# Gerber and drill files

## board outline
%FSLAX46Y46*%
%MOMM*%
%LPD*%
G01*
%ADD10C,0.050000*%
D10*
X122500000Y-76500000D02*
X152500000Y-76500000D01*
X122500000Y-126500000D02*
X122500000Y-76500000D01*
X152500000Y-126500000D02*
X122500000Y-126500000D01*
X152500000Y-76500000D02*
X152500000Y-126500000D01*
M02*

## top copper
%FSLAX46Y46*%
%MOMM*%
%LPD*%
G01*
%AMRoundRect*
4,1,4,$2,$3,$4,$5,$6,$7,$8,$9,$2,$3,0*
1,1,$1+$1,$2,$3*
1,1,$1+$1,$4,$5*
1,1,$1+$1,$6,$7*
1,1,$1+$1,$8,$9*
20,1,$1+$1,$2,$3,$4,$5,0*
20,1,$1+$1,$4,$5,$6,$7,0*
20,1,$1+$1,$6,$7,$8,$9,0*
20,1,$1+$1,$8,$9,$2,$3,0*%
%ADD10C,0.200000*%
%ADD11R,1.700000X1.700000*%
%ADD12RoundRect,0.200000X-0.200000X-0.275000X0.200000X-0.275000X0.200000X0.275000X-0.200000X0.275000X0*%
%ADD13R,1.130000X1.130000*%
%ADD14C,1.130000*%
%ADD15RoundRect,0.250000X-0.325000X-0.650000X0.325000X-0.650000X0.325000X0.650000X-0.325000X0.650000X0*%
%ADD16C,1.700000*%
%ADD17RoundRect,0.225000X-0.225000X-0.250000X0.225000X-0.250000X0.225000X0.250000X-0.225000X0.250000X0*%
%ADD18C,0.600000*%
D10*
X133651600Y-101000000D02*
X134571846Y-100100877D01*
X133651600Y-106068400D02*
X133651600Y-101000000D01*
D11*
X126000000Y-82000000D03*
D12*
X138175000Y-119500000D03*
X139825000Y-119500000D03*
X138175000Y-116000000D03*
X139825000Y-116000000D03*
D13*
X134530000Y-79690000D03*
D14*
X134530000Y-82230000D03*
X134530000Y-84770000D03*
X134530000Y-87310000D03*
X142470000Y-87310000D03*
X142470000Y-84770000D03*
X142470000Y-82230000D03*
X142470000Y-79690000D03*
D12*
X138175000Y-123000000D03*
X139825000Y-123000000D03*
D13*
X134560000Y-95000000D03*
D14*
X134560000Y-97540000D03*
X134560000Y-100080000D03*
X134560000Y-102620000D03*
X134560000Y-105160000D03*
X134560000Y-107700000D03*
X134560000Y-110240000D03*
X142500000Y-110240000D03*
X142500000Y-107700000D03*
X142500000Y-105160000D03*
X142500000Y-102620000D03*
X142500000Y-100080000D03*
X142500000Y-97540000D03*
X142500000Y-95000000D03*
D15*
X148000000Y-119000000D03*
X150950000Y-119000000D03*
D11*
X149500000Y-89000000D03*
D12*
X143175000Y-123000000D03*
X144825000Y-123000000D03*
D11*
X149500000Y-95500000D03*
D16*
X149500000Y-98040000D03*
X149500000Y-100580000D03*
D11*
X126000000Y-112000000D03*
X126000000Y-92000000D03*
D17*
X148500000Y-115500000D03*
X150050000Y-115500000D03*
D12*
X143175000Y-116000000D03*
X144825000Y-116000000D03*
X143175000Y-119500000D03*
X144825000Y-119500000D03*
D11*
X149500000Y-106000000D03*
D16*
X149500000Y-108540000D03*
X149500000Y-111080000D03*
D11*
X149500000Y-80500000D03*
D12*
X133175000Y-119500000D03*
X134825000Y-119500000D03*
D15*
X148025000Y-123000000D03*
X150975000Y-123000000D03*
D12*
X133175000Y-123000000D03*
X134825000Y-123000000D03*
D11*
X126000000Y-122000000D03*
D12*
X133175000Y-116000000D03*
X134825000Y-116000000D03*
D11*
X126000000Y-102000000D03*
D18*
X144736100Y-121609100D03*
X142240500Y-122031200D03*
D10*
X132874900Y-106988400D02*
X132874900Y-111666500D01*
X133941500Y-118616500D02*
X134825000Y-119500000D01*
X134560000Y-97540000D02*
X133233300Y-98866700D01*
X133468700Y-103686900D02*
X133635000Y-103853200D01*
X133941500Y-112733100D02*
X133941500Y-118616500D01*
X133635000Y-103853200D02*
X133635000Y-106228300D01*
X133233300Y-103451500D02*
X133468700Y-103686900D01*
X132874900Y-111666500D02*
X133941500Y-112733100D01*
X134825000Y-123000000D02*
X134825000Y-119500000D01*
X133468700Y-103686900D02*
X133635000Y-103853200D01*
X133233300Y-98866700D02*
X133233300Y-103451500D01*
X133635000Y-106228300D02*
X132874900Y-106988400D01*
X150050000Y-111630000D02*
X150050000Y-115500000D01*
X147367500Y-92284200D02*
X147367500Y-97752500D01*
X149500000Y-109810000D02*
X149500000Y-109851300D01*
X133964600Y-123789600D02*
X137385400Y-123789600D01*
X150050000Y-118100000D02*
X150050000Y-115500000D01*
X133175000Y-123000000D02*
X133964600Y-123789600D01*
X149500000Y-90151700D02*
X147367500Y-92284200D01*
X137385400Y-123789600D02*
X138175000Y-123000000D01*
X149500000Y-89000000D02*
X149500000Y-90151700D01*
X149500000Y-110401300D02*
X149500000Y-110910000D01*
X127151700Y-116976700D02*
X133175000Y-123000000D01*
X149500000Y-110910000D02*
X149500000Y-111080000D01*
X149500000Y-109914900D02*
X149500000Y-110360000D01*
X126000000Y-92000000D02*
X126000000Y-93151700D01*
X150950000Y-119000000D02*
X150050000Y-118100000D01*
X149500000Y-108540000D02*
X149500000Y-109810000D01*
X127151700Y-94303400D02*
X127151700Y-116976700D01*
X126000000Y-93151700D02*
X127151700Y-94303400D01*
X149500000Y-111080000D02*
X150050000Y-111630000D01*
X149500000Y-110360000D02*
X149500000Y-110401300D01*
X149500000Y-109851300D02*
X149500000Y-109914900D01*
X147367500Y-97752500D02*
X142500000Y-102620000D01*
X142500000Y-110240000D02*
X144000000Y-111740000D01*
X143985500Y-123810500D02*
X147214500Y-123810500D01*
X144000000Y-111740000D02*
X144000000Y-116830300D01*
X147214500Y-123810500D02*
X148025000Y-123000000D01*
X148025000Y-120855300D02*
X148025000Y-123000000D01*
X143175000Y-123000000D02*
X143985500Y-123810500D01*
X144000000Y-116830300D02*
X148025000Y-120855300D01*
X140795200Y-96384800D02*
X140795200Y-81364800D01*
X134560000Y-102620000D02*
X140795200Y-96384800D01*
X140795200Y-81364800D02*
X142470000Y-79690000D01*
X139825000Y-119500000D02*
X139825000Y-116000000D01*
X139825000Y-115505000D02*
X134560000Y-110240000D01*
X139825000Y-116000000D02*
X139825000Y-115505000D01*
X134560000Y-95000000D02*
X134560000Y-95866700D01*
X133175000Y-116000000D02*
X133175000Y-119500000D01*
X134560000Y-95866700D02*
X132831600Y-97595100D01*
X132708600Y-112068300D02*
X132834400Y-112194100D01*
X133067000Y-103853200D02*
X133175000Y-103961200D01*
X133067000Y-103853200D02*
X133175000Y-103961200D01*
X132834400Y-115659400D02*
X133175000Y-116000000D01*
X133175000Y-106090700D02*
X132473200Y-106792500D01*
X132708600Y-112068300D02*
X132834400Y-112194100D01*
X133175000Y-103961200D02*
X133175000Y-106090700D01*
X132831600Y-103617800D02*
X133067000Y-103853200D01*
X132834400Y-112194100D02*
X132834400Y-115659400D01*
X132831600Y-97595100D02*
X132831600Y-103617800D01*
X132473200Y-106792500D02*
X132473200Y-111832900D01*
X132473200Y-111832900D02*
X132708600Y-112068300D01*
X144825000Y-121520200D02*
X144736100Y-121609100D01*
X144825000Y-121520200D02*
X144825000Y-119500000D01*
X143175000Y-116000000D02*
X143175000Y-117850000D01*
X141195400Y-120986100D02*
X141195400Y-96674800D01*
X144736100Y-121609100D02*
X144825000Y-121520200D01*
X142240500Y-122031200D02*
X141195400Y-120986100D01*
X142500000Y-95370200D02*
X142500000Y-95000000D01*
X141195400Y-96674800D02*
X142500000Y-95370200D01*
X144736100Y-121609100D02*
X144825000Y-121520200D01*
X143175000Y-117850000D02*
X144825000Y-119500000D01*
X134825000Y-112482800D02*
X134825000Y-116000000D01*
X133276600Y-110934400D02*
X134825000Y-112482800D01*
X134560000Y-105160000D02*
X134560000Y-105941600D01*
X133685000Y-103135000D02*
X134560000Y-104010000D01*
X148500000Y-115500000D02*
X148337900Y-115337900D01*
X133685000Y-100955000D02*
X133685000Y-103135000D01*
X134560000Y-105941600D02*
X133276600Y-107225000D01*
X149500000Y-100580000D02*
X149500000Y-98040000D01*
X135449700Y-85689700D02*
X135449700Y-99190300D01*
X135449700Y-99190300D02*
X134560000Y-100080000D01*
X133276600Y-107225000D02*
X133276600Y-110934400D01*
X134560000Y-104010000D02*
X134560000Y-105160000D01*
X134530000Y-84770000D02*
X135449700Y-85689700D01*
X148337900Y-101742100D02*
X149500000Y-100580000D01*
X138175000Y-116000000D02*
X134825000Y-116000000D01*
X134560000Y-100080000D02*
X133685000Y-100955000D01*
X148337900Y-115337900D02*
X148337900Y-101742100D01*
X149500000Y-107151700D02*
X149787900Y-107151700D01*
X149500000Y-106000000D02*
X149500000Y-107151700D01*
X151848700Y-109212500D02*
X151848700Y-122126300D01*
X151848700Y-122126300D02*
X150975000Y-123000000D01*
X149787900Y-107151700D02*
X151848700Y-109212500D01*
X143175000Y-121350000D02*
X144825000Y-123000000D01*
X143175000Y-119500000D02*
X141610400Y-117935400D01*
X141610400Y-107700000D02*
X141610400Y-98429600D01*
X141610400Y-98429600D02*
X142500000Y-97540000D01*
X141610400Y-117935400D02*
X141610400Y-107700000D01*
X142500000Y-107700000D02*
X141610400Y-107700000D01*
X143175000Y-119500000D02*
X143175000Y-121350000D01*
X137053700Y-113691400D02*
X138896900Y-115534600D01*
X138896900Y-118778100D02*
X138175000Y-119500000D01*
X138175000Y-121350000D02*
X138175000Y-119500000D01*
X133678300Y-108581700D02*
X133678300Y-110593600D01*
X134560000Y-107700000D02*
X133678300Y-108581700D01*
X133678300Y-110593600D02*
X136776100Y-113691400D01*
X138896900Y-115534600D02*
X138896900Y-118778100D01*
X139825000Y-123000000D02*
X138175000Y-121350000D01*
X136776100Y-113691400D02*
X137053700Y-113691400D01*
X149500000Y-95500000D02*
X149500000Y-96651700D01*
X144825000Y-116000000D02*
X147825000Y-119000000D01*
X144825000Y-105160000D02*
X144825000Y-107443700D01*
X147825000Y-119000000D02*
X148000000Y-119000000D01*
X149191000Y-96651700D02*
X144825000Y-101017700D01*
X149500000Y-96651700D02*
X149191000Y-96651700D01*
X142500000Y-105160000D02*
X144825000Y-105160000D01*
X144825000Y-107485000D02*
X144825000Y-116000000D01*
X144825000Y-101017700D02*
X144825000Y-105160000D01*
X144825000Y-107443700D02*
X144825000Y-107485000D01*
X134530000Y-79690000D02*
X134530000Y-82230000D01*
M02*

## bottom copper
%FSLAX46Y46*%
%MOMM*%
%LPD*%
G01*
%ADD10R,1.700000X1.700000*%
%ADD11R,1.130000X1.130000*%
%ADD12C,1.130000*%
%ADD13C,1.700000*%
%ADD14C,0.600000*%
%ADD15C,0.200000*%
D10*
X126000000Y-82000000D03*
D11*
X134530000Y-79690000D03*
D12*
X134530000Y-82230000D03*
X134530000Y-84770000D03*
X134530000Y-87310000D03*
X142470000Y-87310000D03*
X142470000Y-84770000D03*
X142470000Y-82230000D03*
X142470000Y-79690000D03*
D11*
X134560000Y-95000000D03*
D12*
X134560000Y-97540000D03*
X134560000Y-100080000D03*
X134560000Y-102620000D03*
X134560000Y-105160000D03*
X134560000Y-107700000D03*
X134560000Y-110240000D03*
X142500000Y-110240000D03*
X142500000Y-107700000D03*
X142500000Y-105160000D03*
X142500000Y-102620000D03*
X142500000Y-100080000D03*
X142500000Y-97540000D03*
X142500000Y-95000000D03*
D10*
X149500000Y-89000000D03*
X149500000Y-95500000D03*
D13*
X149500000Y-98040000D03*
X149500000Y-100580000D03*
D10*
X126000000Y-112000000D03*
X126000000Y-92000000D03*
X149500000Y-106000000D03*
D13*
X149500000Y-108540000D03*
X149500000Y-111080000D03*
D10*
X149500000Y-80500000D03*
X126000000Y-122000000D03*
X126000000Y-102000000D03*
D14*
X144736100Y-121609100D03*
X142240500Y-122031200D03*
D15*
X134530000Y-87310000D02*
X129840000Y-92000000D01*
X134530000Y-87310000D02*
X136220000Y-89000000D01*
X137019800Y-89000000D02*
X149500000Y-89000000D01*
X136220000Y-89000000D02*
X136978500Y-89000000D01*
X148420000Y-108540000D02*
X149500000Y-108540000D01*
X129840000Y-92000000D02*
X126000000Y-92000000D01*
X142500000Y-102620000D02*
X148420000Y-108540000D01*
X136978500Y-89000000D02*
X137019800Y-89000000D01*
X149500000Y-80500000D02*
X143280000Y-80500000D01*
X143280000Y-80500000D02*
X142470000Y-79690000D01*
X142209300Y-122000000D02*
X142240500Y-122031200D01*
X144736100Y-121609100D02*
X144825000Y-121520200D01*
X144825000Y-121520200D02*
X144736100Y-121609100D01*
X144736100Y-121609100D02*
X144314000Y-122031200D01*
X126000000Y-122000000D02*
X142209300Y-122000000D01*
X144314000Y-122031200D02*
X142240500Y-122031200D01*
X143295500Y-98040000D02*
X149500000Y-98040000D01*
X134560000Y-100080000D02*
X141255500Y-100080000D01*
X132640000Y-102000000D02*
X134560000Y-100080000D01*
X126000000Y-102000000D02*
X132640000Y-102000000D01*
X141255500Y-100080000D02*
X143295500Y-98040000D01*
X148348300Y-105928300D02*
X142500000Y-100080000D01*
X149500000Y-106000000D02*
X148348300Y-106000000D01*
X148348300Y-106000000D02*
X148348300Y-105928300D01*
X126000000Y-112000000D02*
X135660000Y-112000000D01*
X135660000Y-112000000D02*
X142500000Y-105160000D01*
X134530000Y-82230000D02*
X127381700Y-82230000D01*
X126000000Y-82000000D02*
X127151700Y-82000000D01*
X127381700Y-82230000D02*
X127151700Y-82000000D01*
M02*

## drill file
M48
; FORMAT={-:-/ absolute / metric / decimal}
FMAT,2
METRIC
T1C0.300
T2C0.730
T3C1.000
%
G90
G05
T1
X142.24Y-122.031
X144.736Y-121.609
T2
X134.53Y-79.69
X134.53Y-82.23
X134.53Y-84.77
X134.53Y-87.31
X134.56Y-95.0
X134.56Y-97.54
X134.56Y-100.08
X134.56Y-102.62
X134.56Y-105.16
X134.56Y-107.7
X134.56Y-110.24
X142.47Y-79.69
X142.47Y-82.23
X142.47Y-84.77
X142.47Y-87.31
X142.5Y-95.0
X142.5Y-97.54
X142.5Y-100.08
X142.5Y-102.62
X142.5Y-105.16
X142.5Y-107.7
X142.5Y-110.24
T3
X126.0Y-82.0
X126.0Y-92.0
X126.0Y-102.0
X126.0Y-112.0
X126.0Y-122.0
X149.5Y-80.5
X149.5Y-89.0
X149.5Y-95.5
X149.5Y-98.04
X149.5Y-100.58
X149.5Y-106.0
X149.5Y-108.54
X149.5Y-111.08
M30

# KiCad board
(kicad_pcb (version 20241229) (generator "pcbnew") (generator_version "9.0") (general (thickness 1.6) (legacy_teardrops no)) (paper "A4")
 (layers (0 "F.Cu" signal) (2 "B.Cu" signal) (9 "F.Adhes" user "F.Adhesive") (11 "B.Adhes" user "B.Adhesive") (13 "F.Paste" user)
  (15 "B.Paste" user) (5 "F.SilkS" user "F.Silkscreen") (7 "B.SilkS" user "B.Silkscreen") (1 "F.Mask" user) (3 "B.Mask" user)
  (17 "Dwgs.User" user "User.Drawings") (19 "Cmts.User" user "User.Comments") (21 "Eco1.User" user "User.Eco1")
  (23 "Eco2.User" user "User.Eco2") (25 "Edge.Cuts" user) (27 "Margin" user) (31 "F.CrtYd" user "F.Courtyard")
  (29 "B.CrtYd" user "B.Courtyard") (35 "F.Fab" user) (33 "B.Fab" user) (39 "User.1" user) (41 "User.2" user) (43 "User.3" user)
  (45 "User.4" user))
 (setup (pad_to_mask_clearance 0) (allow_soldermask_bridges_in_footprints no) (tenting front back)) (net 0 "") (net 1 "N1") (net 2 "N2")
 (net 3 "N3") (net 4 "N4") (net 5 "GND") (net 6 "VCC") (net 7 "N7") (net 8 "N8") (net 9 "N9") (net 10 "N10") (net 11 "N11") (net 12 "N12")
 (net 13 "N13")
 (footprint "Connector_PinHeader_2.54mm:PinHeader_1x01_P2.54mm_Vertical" (layer "F.Cu") (at 126 82)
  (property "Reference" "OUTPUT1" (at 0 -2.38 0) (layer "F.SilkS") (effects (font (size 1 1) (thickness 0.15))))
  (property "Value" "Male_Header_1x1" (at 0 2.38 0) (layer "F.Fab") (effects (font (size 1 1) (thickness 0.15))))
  (pad "1" thru_hole rect (at 0 0) (size 1.7 1.7) (drill 1) (layers "*.Cu" "*.Mask") (remove_unused_layers no) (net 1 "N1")))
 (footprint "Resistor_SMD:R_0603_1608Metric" (layer "F.Cu") (at 139 119.5)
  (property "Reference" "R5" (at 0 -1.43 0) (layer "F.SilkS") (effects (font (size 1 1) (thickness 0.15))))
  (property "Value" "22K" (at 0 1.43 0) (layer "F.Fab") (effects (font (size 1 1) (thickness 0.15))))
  (pad "1" smd roundrect (at -0.825 0) (size 0.8 0.95) (layers "F.Cu" "F.Mask" "F.Paste") (roundrect_rratio 0.25) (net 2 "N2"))
  (pad "2" smd roundrect (at 0.825 0) (size 0.8 0.95) (layers "F.Cu" "F.Mask" "F.Paste") (roundrect_rratio 0.25) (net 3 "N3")))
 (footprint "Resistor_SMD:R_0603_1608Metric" (layer "F.Cu") (at 139 116)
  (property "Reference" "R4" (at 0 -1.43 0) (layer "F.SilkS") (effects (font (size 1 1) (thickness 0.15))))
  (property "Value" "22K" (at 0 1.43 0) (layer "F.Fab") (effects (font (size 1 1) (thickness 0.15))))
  (pad "1" smd roundrect (at -0.825 0) (size 0.8 0.95) (layers "F.Cu" "F.Mask" "F.Paste") (roundrect_rratio 0.25) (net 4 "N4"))
  (pad "2" smd roundrect (at 0.825 0) (size 0.8 0.95) (layers "F.Cu" "F.Mask" "F.Paste") (roundrect_rratio 0.25) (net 3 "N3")))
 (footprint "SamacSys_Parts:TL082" (layer "F.Cu") (at 138.5 83.5)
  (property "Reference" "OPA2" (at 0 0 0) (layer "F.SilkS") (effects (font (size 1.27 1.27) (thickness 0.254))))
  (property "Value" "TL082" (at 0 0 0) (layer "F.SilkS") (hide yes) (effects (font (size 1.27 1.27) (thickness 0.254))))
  (pad "1" thru_hole rect (at -3.97 -3.81) (size 1.13 1.13) (drill 0.73) (layers "*.Cu" "*.Mask") (remove_unused_layers no) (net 1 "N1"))
  (pad "2" thru_hole circle (at -3.97 -1.27) (size 1.13 1.13) (drill 0.73) (layers "*.Cu" "*.Mask") (remove_unused_layers no) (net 1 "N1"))
  (pad "3" thru_hole circle (at -3.97 1.27) (size 1.13 1.13) (drill 0.73) (layers "*.Cu" "*.Mask") (remove_unused_layers no) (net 4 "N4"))
  (pad "4" thru_hole circle (at -3.97 3.81) (size 1.13 1.13) (drill 0.73) (layers "*.Cu" "*.Mask") (remove_unused_layers no) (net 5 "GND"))
  (pad "5" thru_hole circle (at 3.97 3.81) (size 1.13 1.13) (drill 0.73) (layers "*.Cu" "*.Mask") (remove_unused_layers no))
  (pad "6" thru_hole circle (at 3.97 1.27) (size 1.13 1.13) (drill 0.73) (layers "*.Cu" "*.Mask") (remove_unused_layers no))
  (pad "7" thru_hole circle (at 3.97 -1.27) (size 1.13 1.13) (drill 0.73) (layers "*.Cu" "*.Mask") (remove_unused_layers no))
  (pad "8" thru_hole circle (at 3.97 -3.81) (size 1.13 1.13) (drill 0.73) (layers "*.Cu" "*.Mask") (remove_unused_layers no) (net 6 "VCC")))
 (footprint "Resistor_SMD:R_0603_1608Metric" (layer "F.Cu") (at 139 123)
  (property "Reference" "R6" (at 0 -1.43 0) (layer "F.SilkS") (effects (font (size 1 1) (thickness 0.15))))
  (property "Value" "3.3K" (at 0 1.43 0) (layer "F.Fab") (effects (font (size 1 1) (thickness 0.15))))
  (pad "1" smd roundrect (at -0.825 0) (size 0.8 0.95) (layers "F.Cu" "F.Mask" "F.Paste") (roundrect_rratio 0.25) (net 5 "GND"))
  (pad "2" smd roundrect (at 0.825 0) (size 0.8 0.95) (layers "F.Cu" "F.Mask" "F.Paste") (roundrect_rratio 0.25) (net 2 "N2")))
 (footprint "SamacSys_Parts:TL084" (layer "F.Cu") (at 138.53 102.62)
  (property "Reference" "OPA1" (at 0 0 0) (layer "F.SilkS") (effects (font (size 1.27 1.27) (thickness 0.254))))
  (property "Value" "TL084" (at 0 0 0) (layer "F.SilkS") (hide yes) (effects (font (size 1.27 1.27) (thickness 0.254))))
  (pad "1" thru_hole rect (at -3.97 -7.62) (size 1.13 1.13) (drill 0.73) (layers "*.Cu" "*.Mask") (remove_unused_layers no) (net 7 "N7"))
  (pad "2" thru_hole circle (at -3.97 -5.08) (size 1.13 1.13) (drill 0.73) (layers "*.Cu" "*.Mask") (remove_unused_layers no) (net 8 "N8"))
  (pad "3" thru_hole circle (at -3.97 -2.54) (size 1.13 1.13) (drill 0.73) (layers "*.Cu" "*.Mask") (remove_unused_layers no) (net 4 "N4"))
  (pad "4" thru_hole circle (at -3.97 0) (size 1.13 1.13) (drill 0.73) (layers "*.Cu" "*.Mask") (remove_unused_layers no) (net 6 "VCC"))
  (pad "5" thru_hole circle (at -3.97 2.54) (size 1.13 1.13) (drill 0.73) (layers "*.Cu" "*.Mask") (remove_unused_layers no) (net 4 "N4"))
  (pad "6" thru_hole circle (at -3.97 5.08) (size 1.13 1.13) (drill 0.73) (layers "*.Cu" "*.Mask") (remove_unused_layers no) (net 2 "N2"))
  (pad "7" thru_hole circle (at -3.97 7.62) (size 1.13 1.13) (drill 0.73) (layers "*.Cu" "*.Mask") (remove_unused_layers no) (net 3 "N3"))
  (pad "8" thru_hole circle (at 3.97 7.62) (size 1.13 1.13) (drill 0.73) (layers "*.Cu" "*.Mask") (remove_unused_layers no) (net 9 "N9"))
  (pad "9" thru_hole circle (at 3.97 5.08) (size 1.13 1.13) (drill 0.73) (layers "*.Cu" "*.Mask") (remove_unused_layers no) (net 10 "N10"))
  (pad "10" thru_hole circle (at 3.97 2.54) (size 1.13 1.13) (drill 0.73) (layers "*.Cu" "*.Mask") (remove_unused_layers no) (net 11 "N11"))
  (pad "11" thru_hole circle (at 3.97 0) (size 1.13 1.13) (drill 0.73) (layers "*.Cu" "*.Mask") (remove_unused_layers no) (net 5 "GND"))
  (pad "12" thru_hole circle (at 3.97 -2.54) (size 1.13 1.13) (drill 0.73) (layers "*.Cu" "*.Mask") (remove_unused_layers no) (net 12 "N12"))
  (pad "13" thru_hole circle (at 3.97 -5.08) (size 1.13 1.13) (drill 0.73) (layers "*.Cu" "*.Mask") (remove_unused_layers no) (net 10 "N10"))
  (pad "14" thru_hole circle (at 3.97 -7.62) (size 1.13 1.13) (drill 0.73) (layers "*.Cu" "*.Mask") (remove_unused_layers no) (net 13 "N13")))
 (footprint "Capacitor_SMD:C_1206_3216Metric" (layer "F.Cu") (at 149.475 119)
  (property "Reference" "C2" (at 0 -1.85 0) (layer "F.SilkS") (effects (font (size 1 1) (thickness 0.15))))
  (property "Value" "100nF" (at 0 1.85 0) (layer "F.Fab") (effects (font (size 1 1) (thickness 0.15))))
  (pad "1" smd roundrect (at -1.475 0) (size 1.15 1.8) (layers "F.Cu" "F.Mask" "F.Paste") (roundrect_rratio 0.217391) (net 11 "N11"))
  (pad "2" smd roundrect (at 1.475 0) (size 1.15 1.8) (layers "F.Cu" "F.Mask" "F.Paste") (roundrect_rratio 0.217391) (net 5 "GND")))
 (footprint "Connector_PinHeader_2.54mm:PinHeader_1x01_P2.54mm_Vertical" (layer "F.Cu") (at 149.5 89)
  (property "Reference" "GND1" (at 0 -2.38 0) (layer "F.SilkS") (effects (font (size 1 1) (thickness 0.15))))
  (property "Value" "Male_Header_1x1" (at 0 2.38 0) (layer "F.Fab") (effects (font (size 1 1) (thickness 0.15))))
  (pad "1" thru_hole rect (at 0 0) (size 1.7 1.7) (drill 1) (layers "*.Cu" "*.Mask") (remove_unused_layers no) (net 5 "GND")))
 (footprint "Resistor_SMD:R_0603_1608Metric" (layer "F.Cu") (at 144 123)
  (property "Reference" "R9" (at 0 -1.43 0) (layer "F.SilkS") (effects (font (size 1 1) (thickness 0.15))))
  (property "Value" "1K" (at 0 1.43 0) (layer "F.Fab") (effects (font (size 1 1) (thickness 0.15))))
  (pad "1" smd roundrect (at -0.825 0) (size 0.8 0.95) (layers "F.Cu" "F.Mask" "F.Paste") (roundrect_rratio 0.25) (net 9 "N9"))
  (pad "2" smd roundrect (at 0.825 0) (size 0.8 0.95) (layers "F.Cu" "F.Mask" "F.Paste") (roundrect_rratio 0.25) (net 10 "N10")))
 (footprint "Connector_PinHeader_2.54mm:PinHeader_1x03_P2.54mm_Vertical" (layer "F.Cu") (at 149.5 95.5)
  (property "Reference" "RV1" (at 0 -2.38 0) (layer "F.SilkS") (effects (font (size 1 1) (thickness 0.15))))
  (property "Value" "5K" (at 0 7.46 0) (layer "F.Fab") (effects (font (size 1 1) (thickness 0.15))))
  (pad "1" thru_hole rect (at 0 0) (size 1.7 1.7) (drill 1) (layers "*.Cu" "*.Mask") (remove_unused_layers no) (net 11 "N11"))
  (pad "2" thru_hole circle (at 0 2.54) (size 1.7 1.7) (drill 1) (layers "*.Cu" "*.Mask") (remove_unused_layers no) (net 4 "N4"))
  (pad "3" thru_hole circle (at 0 5.08) (size 1.7 1.7) (drill 1) (layers "*.Cu" "*.Mask") (remove_unused_layers no) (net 4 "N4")))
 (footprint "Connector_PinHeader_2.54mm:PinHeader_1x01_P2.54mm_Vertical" (layer "F.Cu") (at 126 112)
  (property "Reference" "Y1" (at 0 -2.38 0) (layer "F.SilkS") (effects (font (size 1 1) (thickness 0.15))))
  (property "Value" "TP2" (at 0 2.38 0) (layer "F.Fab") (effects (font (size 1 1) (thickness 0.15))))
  (pad "1" thru_hole rect (at 0 0) (size 1.7 1.7) (drill 1) (layers "*.Cu" "*.Mask") (remove_unused_layers no) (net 11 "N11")))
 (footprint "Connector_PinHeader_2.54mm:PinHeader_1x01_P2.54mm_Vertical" (layer "F.Cu") (at 126 92)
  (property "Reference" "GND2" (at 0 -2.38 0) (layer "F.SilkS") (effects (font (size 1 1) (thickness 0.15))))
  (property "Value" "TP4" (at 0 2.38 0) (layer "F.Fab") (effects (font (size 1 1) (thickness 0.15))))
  (pad "1" thru_hole rect (at 0 0) (size 1.7 1.7) (drill 1) (layers "*.Cu" "*.Mask") (remove_unused_layers no) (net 5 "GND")))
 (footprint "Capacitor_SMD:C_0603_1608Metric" (layer "F.Cu") (at 149.275 115.5)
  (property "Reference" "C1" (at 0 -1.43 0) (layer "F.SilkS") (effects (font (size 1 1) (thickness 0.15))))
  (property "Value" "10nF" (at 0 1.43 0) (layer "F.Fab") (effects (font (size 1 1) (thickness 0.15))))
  (pad "1" smd roundrect (at -0.775 0) (size 0.9 0.95) (layers "F.Cu" "F.Mask" "F.Paste") (roundrect_rratio 0.25) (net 4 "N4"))
  (pad "2" smd roundrect (at 0.775 0) (size 0.9 0.95) (layers "F.Cu" "F.Mask" "F.Paste") (roundrect_rratio 0.25) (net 5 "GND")))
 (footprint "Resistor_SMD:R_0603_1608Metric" (layer "F.Cu") (at 144 116)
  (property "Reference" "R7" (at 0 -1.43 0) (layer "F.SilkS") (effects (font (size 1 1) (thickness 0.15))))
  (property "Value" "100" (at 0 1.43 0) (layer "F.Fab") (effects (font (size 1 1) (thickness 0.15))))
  (pad "1" smd roundrect (at -0.825 0) (size 0.8 0.95) (layers "F.Cu" "F.Mask" "F.Paste") (roundrect_rratio 0.25) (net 13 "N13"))
  (pad "2" smd roundrect (at 0.825 0) (size 0.8 0.95) (layers "F.Cu" "F.Mask" "F.Paste") (roundrect_rratio 0.25) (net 11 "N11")))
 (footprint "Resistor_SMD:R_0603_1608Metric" (layer "F.Cu") (at 144 119.5)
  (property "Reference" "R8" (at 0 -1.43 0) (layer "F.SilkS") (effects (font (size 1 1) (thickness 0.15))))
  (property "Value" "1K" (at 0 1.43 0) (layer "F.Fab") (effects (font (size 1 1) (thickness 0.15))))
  (pad "1" smd roundrect (at -0.825 0) (size 0.8 0.95) (layers "F.Cu" "F.Mask" "F.Paste") (roundrect_rratio 0.25) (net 10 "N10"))
  (pad "2" smd roundrect (at 0.825 0) (size 0.8 0.95) (layers "F.Cu" "F.Mask" "F.Paste") (roundrect_rratio 0.25) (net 13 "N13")))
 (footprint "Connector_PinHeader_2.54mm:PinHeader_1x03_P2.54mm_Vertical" (layer "F.Cu") (at 149.5 106)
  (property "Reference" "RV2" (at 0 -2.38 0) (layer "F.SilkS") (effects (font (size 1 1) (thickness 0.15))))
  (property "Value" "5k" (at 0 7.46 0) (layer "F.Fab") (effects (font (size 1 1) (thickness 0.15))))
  (pad "1" thru_hole rect (at 0 0) (size 1.7 1.7) (drill 1) (layers "*.Cu" "*.Mask") (remove_unused_layers no) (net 12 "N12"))
  (pad "2" thru_hole circle (at 0 2.54) (size 1.7 1.7) (drill 1) (layers "*.Cu" "*.Mask") (remove_unused_layers no) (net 5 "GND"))
  (pad "3" thru_hole circle (at 0 5.08) (size 1.7 1.7) (drill 1) (layers "*.Cu" "*.Mask") (remove_unused_layers no) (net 5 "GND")))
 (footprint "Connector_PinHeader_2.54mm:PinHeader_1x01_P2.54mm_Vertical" (layer "F.Cu") (at 149.5 80.5)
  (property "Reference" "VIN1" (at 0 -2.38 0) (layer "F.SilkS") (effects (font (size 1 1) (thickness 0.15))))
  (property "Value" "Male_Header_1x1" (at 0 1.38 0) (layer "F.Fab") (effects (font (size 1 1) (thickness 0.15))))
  (pad "1" thru_hole rect (at 0 0) (size 1.7 1.7) (drill 1) (layers "*.Cu" "*.Mask") (remove_unused_layers no) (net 6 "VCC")))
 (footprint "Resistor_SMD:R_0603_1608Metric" (layer "F.Cu") (at 134 119.5)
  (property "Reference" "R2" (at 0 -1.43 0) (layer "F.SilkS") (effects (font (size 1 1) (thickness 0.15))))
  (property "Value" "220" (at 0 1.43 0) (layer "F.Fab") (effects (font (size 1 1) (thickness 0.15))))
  (pad "1" smd roundrect (at -0.825 0) (size 0.8 0.95) (layers "F.Cu" "F.Mask" "F.Paste") (roundrect_rratio 0.25) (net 7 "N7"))
  (pad "2" smd roundrect (at 0.825 0) (size 0.8 0.95) (layers "F.Cu" "F.Mask" "F.Paste") (roundrect_rratio 0.25) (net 8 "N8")))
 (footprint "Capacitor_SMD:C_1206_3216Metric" (layer "F.Cu") (at 149.5 123)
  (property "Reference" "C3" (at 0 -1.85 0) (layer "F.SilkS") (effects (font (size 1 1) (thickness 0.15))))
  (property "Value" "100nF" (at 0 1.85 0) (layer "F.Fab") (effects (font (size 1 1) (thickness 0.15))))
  (pad "1" smd roundrect (at -1.475 0) (size 1.15 1.8) (layers "F.Cu" "F.Mask" "F.Paste") (roundrect_rratio 0.217391) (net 9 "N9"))
  (pad "2" smd roundrect (at 1.475 0) (size 1.15 1.8) (layers "F.Cu" "F.Mask" "F.Paste") (roundrect_rratio 0.217391) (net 12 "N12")))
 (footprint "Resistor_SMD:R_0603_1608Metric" (layer "F.Cu") (at 134 123)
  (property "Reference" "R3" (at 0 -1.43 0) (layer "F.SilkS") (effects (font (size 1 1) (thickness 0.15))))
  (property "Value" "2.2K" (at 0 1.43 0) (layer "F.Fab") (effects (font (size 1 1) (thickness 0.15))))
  (pad "1" smd roundrect (at -0.825 0) (size 0.8 0.95) (layers "F.Cu" "F.Mask" "F.Paste") (roundrect_rratio 0.25) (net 5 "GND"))
  (pad "2" smd roundrect (at 0.825 0) (size 0.8 0.95) (layers "F.Cu" "F.Mask" "F.Paste") (roundrect_rratio 0.25) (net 8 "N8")))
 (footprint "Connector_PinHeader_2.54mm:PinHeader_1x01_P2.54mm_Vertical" (layer "F.Cu") (at 126 122)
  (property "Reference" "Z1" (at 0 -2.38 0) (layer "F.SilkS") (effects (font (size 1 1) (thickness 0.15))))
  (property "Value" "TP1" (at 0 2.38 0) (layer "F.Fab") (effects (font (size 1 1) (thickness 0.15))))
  (pad "1" thru_hole rect (at 0 0) (size 1.7 1.7) (drill 1) (layers "*.Cu" "*.Mask") (remove_unused_layers no) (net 13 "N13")))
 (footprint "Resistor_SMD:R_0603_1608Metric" (layer "F.Cu") (at 134 116)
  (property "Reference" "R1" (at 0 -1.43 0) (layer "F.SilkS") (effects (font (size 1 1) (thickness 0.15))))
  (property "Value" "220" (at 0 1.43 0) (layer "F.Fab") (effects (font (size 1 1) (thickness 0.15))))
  (pad "1" smd roundrect (at -0.825 0) (size 0.8 0.95) (layers "F.Cu" "F.Mask" "F.Paste") (roundrect_rratio 0.25) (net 7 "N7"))
  (pad "2" smd roundrect (at 0.825 0) (size 0.8 0.95) (layers "F.Cu" "F.Mask" "F.Paste") (roundrect_rratio 0.25) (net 4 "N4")))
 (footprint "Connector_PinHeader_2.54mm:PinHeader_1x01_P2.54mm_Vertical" (layer "F.Cu") (at 126 102)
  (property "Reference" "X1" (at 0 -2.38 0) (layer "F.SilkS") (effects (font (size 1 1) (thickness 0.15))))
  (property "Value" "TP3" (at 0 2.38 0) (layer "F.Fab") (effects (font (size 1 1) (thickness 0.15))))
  (pad "1" thru_hole rect (at 0 0) (size 1.7 1.7) (drill 1) (layers "*.Cu" "*.Mask") (remove_unused_layers no) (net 4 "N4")))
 (gr_line (start 133.6516 101) (end 134.571846 100.100877) (stroke (width 0.2) (type default)) (layer "F.Cu") (net 4))
 (gr_line (start 133.6516 106.0684) (end 133.6516 101) (stroke (width 0.2) (type default)) (layer "F.Cu") (net 4))
 (gr_line (start 122.5 76.5) (end 152.5 76.5) (stroke (width 0.05) (type default)) (layer "Edge.Cuts"))
 (gr_line (start 122.5 126.5) (end 122.5 76.5) (stroke (width 0.05) (type default)) (layer "Edge.Cuts"))
 (gr_line (start 152.5 126.5) (end 122.5 126.5) (stroke (width 0.05) (type default)) (layer "Edge.Cuts"))
 (gr_line (start 152.5 76.5) (end 152.5 126.5) (stroke (width 0.05) (type default)) (layer "Edge.Cuts"))
 (segment (start 132.8749 106.9884) (end 132.8749 111.6665) (width 0.2) (layer "F.Cu") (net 8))
 (segment (start 133.9415 118.6165) (end 134.825 119.5) (width 0.2) (layer "F.Cu") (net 8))
 (segment (start 134.56 97.54) (end 133.2333 98.8667) (width 0.2) (layer "F.Cu") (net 8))
 (segment (start 133.4687 103.6869) (end 133.635 103.8532) (width 0.2) (layer "F.Cu") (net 8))
 (segment (start 133.9415 112.7331) (end 133.9415 118.6165) (width 0.2) (layer "F.Cu") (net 8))
 (segment (start 133.635 103.8532) (end 133.635 106.2283) (width 0.2) (layer "F.Cu") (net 8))
 (segment (start 133.2333 103.4515) (end 133.4687 103.6869) (width 0.2) (layer "F.Cu") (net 8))
 (segment (start 132.8749 111.6665) (end 133.9415 112.7331) (width 0.2) (layer "F.Cu") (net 8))
 (segment (start 134.825 123) (end 134.825 119.5) (width 0.2) (layer "F.Cu") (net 8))
 (segment (start 133.4687 103.6869) (end 133.635 103.8532) (width 0.2) (layer "F.Cu") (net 8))
 (segment (start 133.2333 98.8667) (end 133.2333 103.4515) (width 0.2) (layer "F.Cu") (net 8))
 (segment (start 133.635 106.2283) (end 132.8749 106.9884) (width 0.2) (layer "F.Cu") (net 8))
 (segment (start 150.05 111.63) (end 150.05 115.5) (width 0.2) (layer "F.Cu") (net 5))
 (segment (start 147.3675 92.2842) (end 147.3675 97.7525) (width 0.2) (layer "F.Cu") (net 5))
 (segment (start 149.5 109.81) (end 149.5 109.8513) (width 0.2) (layer "F.Cu") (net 5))
 (segment (start 133.9646 123.7896) (end 137.3854 123.7896) (width 0.2) (layer "F.Cu") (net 5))
 (segment (start 150.05 118.1) (end 150.05 115.5) (width 0.2) (layer "F.Cu") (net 5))
 (segment (start 133.175 123) (end 133.9646 123.7896) (width 0.2) (layer "F.Cu") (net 5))
 (segment (start 149.5 90.1517) (end 147.3675 92.2842) (width 0.2) (layer "F.Cu") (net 5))
 (segment (start 137.3854 123.7896) (end 138.175 123) (width 0.2) (layer "F.Cu") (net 5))
 (segment (start 149.5 89) (end 149.5 90.1517) (width 0.2) (layer "F.Cu") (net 5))
 (segment (start 149.5 110.4013) (end 149.5 110.91) (width 0.2) (layer "F.Cu") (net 5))
 (segment (start 127.1517 116.9767) (end 133.175 123) (width 0.2) (layer "F.Cu") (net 5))
 (segment (start 149.5 110.91) (end 149.5 111.08) (width 0.2) (layer "F.Cu") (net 5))
 (segment (start 149.5 109.9149) (end 149.5 110.36) (width 0.2) (layer "F.Cu") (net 5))
 (segment (start 126 92) (end 126 93.1517) (width 0.2) (layer "F.Cu") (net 5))
 (segment (start 150.95 119) (end 150.05 118.1) (width 0.2) (layer "F.Cu") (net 5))
 (segment (start 149.5 108.54) (end 149.5 109.81) (width 0.2) (layer "F.Cu") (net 5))
 (segment (start 127.1517 94.3034) (end 127.1517 116.9767) (width 0.2) (layer "F.Cu") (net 5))
 (segment (start 126 93.1517) (end 127.1517 94.3034) (width 0.2) (layer "F.Cu") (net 5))
 (segment (start 149.5 111.08) (end 150.05 111.63) (width 0.2) (layer "F.Cu") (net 5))
 (segment (start 149.5 110.36) (end 149.5 110.4013) (width 0.2) (layer "F.Cu") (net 5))
 (segment (start 149.5 109.8513) (end 149.5 109.9149) (width 0.2) (layer "F.Cu") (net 5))
 (segment (start 147.3675 97.7525) (end 142.5 102.62) (width 0.2) (layer "F.Cu") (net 5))
 (segment (start 134.53 87.31) (end 129.84 92) (width 0.2) (layer "B.Cu") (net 5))
 (segment (start 134.53 87.31) (end 136.22 89) (width 0.2) (layer "B.Cu") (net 5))
 (segment (start 137.0198 89) (end 149.5 89) (width 0.2) (layer "B.Cu") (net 5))
 (segment (start 136.22 89) (end 136.9785 89) (width 0.2) (layer "B.Cu") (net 5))
 (segment (start 148.42 108.54) (end 149.5 108.54) (width 0.2) (layer "B.Cu") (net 5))
 (segment (start 129.84 92) (end 126 92) (width 0.2) (layer "B.Cu") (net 5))
 (segment (start 142.5 102.62) (end 148.42 108.54) (width 0.2) (layer "B.Cu") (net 5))
 (segment (start 136.9785 89) (end 137.0198 89) (width 0.2) (layer "B.Cu") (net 5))
 (segment (start 142.5 110.24) (end 144 111.74) (width 0.2) (layer "F.Cu") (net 9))
 (segment (start 143.9855 123.8105) (end 147.2145 123.8105) (width 0.2) (layer "F.Cu") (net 9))
 (segment (start 144 111.74) (end 144 116.8303) (width 0.2) (layer "F.Cu") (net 9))
 (segment (start 147.2145 123.8105) (end 148.025 123) (width 0.2) (layer "F.Cu") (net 9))
 (segment (start 148.025 120.8553) (end 148.025 123) (width 0.2) (layer "F.Cu") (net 9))
 (segment (start 143.175 123) (end 143.9855 123.8105) (width 0.2) (layer "F.Cu") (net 9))
 (segment (start 144 116.8303) (end 148.025 120.8553) (width 0.2) (layer "F.Cu") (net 9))
 (segment (start 140.7952 96.3848) (end 140.7952 81.3648) (width 0.2) (layer "F.Cu") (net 6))
 (segment (start 134.56 102.62) (end 140.7952 96.3848) (width 0.2) (layer "F.Cu") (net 6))
 (segment (start 140.7952 81.3648) (end 142.47 79.69) (width 0.2) (layer "F.Cu") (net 6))
 (segment (start 149.5 80.5) (end 143.28 80.5) (width 0.2) (layer "B.Cu") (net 6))
 (segment (start 143.28 80.5) (end 142.47 79.69) (width 0.2) (layer "B.Cu") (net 6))
 (segment (start 139.825 119.5) (end 139.825 116) (width 0.2) (layer "F.Cu") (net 3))
 (segment (start 139.825 115.505) (end 134.56 110.24) (width 0.2) (layer "F.Cu") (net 3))
 (segment (start 139.825 116) (end 139.825 115.505) (width 0.2) (layer "F.Cu") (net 3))
 (segment (start 134.56 95) (end 134.56 95.8667) (width 0.2) (layer "F.Cu") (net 7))
 (segment (start 133.175 116) (end 133.175 119.5) (width 0.2) (layer "F.Cu") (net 7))
 (segment (start 134.56 95.8667) (end 132.8316 97.5951) (width 0.2) (layer "F.Cu") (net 7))
 (segment (start 132.7086 112.0683) (end 132.8344 112.1941) (width 0.2) (layer "F.Cu") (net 7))
 (segment (start 133.067 103.8532) (end 133.175 103.9612) (width 0.2) (layer "F.Cu") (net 7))
 (segment (start 133.067 103.8532) (end 133.175 103.9612) (width 0.2) (layer "F.Cu") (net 7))
 (segment (start 132.8344 115.6594) (end 133.175 116) (width 0.2) (layer "F.Cu") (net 7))
 (segment (start 133.175 106.0907) (end 132.4732 106.7925) (width 0.2) (layer "F.Cu") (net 7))
 (segment (start 132.7086 112.0683) (end 132.8344 112.1941) (width 0.2) (layer "F.Cu") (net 7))
 (segment (start 133.175 103.9612) (end 133.175 106.0907) (width 0.2) (layer "F.Cu") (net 7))
 (segment (start 132.8316 103.6178) (end 133.067 103.8532) (width 0.2) (layer "F.Cu") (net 7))
 (segment (start 132.8344 112.1941) (end 132.8344 115.6594) (width 0.2) (layer "F.Cu") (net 7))
 (segment (start 132.8316 97.5951) (end 132.8316 103.6178) (width 0.2) (layer "F.Cu") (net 7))
 (segment (start 132.4732 106.7925) (end 132.4732 111.8329) (width 0.2) (layer "F.Cu") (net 7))
 (segment (start 132.4732 111.8329) (end 132.7086 112.0683) (width 0.2) (layer "F.Cu") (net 7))
 (segment (start 144.825 121.5202) (end 144.7361 121.6091) (width 0.2) (layer "F.Cu") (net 13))
 (segment (start 144.825 121.5202) (end 144.825 119.5) (width 0.2) (layer "F.Cu") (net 13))
 (segment (start 143.175 116) (end 143.175 117.85) (width 0.2) (layer "F.Cu") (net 13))
 (segment (start 141.1954 120.9861) (end 141.1954 96.6748) (width 0.2) (layer "F.Cu") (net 13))
 (segment (start 144.7361 121.6091) (end 144.825 121.5202) (width 0.2) (layer "F.Cu") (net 13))
 (segment (start 142.2405 122.0312) (end 141.1954 120.9861) (width 0.2) (layer "F.Cu") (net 13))
 (segment (start 142.5 95.3702) (end 142.5 95) (width 0.2) (layer "F.Cu") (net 13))
 (segment (start 141.1954 96.6748) (end 142.5 95.3702) (width 0.2) (layer "F.Cu") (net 13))
 (segment (start 144.7361 121.6091) (end 144.825 121.5202) (width 0.2) (layer "F.Cu") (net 13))
 (segment (start 143.175 117.85) (end 144.825 119.5) (width 0.2) (layer "F.Cu") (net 13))
 (via (at 144.7361 121.6091) (size 0.6) (drill 0.3) (layers "F.Cu" "B.Cu") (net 13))
 (via (at 142.2405 122.0312) (size 0.6) (drill 0.3) (layers "F.Cu" "B.Cu") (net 13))
 (segment (start 142.2093 122) (end 142.2405 122.0312) (width 0.2) (layer "B.Cu") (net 13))
 (segment (start 144.7361 121.6091) (end 144.825 121.5202) (width 0.2) (layer "B.Cu") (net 13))
 (segment (start 144.825 121.5202) (end 144.7361 121.6091) (width 0.2) (layer "B.Cu") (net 13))
 (segment (start 144.7361 121.6091) (end 144.314 122.0312) (width 0.2) (layer "B.Cu") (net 13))
 (segment (start 126 122) (end 142.2093 122) (width 0.2) (layer "B.Cu") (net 13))
 (segment (start 144.314 122.0312) (end 142.2405 122.0312) (width 0.2) (layer "B.Cu") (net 13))
 (segment (start 134.825 112.4828) (end 134.825 116) (width 0.2) (layer "F.Cu") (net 4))
 (segment (start 133.2766 110.9344) (end 134.825 112.4828) (width 0.2) (layer "F.Cu") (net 4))
 (segment (start 134.56 105.16) (end 134.56 105.9416) (width 0.2) (layer "F.Cu") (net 4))
 (segment (start 133.685 103.135) (end 134.56 104.01) (width 0.2) (layer "F.Cu") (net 4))
 (segment (start 148.5 115.5) (end 148.3379 115.3379) (width 0.2) (layer "F.Cu") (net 4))
 (segment (start 133.685 100.955) (end 133.685 103.135) (width 0.2) (layer "F.Cu") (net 4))
 (segment (start 134.56 105.9416) (end 133.2766 107.225) (width 0.2) (layer "F.Cu") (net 4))
 (segment (start 149.5 100.58) (end 149.5 98.04) (width 0.2) (layer "F.Cu") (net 4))
 (segment (start 135.4497 85.6897) (end 135.4497 99.1903) (width 0.2) (layer "F.Cu") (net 4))
 (segment (start 135.4497 99.1903) (end 134.56 100.08) (width 0.2) (layer "F.Cu") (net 4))
 (segment (start 133.2766 107.225) (end 133.2766 110.9344) (width 0.2) (layer "F.Cu") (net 4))
 (segment (start 134.56 104.01) (end 134.56 105.16) (width 0.2) (layer "F.Cu") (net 4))
 (segment (start 134.53 84.77) (end 135.4497 85.6897) (width 0.2) (layer "F.Cu") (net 4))
 (segment (start 148.3379 101.7421) (end 149.5 100.58) (width 0.2) (layer "F.Cu") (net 4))
 (segment (start 138.175 116) (end 134.825 116) (width 0.2) (layer "F.Cu") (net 4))
 (segment (start 134.56 100.08) (end 133.685 100.955) (width 0.2) (layer "F.Cu") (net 4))
 (segment (start 148.3379 115.3379) (end 148.3379 101.7421) (width 0.2) (layer "F.Cu") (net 4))
 (segment (start 143.2955 98.04) (end 149.5 98.04) (width 0.2) (layer "B.Cu") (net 4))
 (segment (start 134.56 100.08) (end 141.2555 100.08) (width 0.2) (layer "B.Cu") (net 4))
 (segment (start 132.64 102) (end 134.56 100.08) (width 0.2) (layer "B.Cu") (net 4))
 (segment (start 126 102) (end 132.64 102) (width 0.2) (layer "B.Cu") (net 4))
 (segment (start 141.2555 100.08) (end 143.2955 98.04) (width 0.2) (layer "B.Cu") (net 4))
 (segment (start 149.5 107.1517) (end 149.7879 107.1517) (width 0.2) (layer "F.Cu") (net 12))
 (segment (start 149.5 106) (end 149.5 107.1517) (width 0.2) (layer "F.Cu") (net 12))
 (segment (start 151.8487 109.2125) (end 151.8487 122.1263) (width 0.2) (layer "F.Cu") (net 12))
 (segment (start 151.8487 122.1263) (end 150.975 123) (width 0.2) (layer "F.Cu") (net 12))
 (segment (start 149.7879 107.1517) (end 151.8487 109.2125) (width 0.2) (layer "F.Cu") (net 12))
 (segment (start 148.3483 105.9283) (end 142.5 100.08) (width 0.2) (layer "B.Cu") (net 12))
 (segment (start 149.5 106) (end 148.3483 106) (width 0.2) (layer "B.Cu") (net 12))
 (segment (start 148.3483 106) (end 148.3483 105.9283) (width 0.2) (layer "B.Cu") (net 12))
 (segment (start 143.175 121.35) (end 144.825 123) (width 0.2) (layer "F.Cu") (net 10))
 (segment (start 143.175 119.5) (end 141.6104 117.9354) (width 0.2) (layer "F.Cu") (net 10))
 (segment (start 141.6104 107.7) (end 141.6104 98.4296) (width 0.2) (layer "F.Cu") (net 10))
 (segment (start 141.6104 98.4296) (end 142.5 97.54) (width 0.2) (layer "F.Cu") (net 10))
 (segment (start 141.6104 117.9354) (end 141.6104 107.7) (width 0.2) (layer "F.Cu") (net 10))
 (segment (start 142.5 107.7) (end 141.6104 107.7) (width 0.2) (layer "F.Cu") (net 10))
 (segment (start 143.175 119.5) (end 143.175 121.35) (width 0.2) (layer "F.Cu") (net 10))
 (segment (start 137.0537 113.6914) (end 138.8969 115.5346) (width 0.2) (layer "F.Cu") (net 2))
 (segment (start 138.8969 118.7781) (end 138.175 119.5) (width 0.2) (layer "F.Cu") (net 2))
 (segment (start 138.175 121.35) (end 138.175 119.5) (width 0.2) (layer "F.Cu") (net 2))
 (segment (start 133.6783 108.5817) (end 133.6783 110.5936) (width 0.2) (layer "F.Cu") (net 2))
 (segment (start 134.56 107.7) (end 133.6783 108.5817) (width 0.2) (layer "F.Cu") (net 2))
 (segment (start 133.6783 110.5936) (end 136.7761 113.6914) (width 0.2) (layer "F.Cu") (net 2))
 (segment (start 138.8969 115.5346) (end 138.8969 118.7781) (width 0.2) (layer "F.Cu") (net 2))
 (segment (start 139.825 123) (end 138.175 121.35) (width 0.2) (layer "F.Cu") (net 2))
 (segment (start 136.7761 113.6914) (end 137.0537 113.6914) (width 0.2) (layer "F.Cu") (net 2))
 (segment (start 149.5 95.5) (end 149.5 96.6517) (width 0.2) (layer "F.Cu") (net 11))
 (segment (start 144.825 116) (end 147.825 119) (width 0.2) (layer "F.Cu") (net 11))
 (segment (start 144.825 105.16) (end 144.825 107.4437) (width 0.2) (layer "F.Cu") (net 11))
 (segment (start 147.825 119) (end 148 119) (width 0.2) (layer "F.Cu") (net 11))
 (segment (start 149.191 96.6517) (end 144.825 101.0177) (width 0.2) (layer "F.Cu") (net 11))
 (segment (start 149.5 96.6517) (end 149.191 96.6517) (width 0.2) (layer "F.Cu") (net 11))
 (segment (start 142.5 105.16) (end 144.825 105.16) (width 0.2) (layer "F.Cu") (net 11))
 (segment (start 144.825 107.485) (end 144.825 116) (width 0.2) (layer "F.Cu") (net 11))
 (segment (start 144.825 101.0177) (end 144.825 105.16) (width 0.2) (layer "F.Cu") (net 11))
 (segment (start 144.825 107.4437) (end 144.825 107.485) (width 0.2) (layer "F.Cu") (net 11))
 (segment (start 126 112) (end 135.66 112) (width 0.2) (layer "B.Cu") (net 11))
 (segment (start 135.66 112) (end 142.5 105.16) (width 0.2) (layer "B.Cu") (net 11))
 (segment (start 134.53 79.69) (end 134.53 82.23) (width 0.2) (layer "F.Cu") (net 1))
 (segment (start 134.53 82.23) (end 127.3817 82.23) (width 0.2) (layer "B.Cu") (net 1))
 (segment (start 126 82) (end 127.1517 82) (width 0.2) (layer "B.Cu") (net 1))
 (segment (start 127.3817 82.23) (end 127.1517 82) (width 0.2) (layer "B.Cu") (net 1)))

